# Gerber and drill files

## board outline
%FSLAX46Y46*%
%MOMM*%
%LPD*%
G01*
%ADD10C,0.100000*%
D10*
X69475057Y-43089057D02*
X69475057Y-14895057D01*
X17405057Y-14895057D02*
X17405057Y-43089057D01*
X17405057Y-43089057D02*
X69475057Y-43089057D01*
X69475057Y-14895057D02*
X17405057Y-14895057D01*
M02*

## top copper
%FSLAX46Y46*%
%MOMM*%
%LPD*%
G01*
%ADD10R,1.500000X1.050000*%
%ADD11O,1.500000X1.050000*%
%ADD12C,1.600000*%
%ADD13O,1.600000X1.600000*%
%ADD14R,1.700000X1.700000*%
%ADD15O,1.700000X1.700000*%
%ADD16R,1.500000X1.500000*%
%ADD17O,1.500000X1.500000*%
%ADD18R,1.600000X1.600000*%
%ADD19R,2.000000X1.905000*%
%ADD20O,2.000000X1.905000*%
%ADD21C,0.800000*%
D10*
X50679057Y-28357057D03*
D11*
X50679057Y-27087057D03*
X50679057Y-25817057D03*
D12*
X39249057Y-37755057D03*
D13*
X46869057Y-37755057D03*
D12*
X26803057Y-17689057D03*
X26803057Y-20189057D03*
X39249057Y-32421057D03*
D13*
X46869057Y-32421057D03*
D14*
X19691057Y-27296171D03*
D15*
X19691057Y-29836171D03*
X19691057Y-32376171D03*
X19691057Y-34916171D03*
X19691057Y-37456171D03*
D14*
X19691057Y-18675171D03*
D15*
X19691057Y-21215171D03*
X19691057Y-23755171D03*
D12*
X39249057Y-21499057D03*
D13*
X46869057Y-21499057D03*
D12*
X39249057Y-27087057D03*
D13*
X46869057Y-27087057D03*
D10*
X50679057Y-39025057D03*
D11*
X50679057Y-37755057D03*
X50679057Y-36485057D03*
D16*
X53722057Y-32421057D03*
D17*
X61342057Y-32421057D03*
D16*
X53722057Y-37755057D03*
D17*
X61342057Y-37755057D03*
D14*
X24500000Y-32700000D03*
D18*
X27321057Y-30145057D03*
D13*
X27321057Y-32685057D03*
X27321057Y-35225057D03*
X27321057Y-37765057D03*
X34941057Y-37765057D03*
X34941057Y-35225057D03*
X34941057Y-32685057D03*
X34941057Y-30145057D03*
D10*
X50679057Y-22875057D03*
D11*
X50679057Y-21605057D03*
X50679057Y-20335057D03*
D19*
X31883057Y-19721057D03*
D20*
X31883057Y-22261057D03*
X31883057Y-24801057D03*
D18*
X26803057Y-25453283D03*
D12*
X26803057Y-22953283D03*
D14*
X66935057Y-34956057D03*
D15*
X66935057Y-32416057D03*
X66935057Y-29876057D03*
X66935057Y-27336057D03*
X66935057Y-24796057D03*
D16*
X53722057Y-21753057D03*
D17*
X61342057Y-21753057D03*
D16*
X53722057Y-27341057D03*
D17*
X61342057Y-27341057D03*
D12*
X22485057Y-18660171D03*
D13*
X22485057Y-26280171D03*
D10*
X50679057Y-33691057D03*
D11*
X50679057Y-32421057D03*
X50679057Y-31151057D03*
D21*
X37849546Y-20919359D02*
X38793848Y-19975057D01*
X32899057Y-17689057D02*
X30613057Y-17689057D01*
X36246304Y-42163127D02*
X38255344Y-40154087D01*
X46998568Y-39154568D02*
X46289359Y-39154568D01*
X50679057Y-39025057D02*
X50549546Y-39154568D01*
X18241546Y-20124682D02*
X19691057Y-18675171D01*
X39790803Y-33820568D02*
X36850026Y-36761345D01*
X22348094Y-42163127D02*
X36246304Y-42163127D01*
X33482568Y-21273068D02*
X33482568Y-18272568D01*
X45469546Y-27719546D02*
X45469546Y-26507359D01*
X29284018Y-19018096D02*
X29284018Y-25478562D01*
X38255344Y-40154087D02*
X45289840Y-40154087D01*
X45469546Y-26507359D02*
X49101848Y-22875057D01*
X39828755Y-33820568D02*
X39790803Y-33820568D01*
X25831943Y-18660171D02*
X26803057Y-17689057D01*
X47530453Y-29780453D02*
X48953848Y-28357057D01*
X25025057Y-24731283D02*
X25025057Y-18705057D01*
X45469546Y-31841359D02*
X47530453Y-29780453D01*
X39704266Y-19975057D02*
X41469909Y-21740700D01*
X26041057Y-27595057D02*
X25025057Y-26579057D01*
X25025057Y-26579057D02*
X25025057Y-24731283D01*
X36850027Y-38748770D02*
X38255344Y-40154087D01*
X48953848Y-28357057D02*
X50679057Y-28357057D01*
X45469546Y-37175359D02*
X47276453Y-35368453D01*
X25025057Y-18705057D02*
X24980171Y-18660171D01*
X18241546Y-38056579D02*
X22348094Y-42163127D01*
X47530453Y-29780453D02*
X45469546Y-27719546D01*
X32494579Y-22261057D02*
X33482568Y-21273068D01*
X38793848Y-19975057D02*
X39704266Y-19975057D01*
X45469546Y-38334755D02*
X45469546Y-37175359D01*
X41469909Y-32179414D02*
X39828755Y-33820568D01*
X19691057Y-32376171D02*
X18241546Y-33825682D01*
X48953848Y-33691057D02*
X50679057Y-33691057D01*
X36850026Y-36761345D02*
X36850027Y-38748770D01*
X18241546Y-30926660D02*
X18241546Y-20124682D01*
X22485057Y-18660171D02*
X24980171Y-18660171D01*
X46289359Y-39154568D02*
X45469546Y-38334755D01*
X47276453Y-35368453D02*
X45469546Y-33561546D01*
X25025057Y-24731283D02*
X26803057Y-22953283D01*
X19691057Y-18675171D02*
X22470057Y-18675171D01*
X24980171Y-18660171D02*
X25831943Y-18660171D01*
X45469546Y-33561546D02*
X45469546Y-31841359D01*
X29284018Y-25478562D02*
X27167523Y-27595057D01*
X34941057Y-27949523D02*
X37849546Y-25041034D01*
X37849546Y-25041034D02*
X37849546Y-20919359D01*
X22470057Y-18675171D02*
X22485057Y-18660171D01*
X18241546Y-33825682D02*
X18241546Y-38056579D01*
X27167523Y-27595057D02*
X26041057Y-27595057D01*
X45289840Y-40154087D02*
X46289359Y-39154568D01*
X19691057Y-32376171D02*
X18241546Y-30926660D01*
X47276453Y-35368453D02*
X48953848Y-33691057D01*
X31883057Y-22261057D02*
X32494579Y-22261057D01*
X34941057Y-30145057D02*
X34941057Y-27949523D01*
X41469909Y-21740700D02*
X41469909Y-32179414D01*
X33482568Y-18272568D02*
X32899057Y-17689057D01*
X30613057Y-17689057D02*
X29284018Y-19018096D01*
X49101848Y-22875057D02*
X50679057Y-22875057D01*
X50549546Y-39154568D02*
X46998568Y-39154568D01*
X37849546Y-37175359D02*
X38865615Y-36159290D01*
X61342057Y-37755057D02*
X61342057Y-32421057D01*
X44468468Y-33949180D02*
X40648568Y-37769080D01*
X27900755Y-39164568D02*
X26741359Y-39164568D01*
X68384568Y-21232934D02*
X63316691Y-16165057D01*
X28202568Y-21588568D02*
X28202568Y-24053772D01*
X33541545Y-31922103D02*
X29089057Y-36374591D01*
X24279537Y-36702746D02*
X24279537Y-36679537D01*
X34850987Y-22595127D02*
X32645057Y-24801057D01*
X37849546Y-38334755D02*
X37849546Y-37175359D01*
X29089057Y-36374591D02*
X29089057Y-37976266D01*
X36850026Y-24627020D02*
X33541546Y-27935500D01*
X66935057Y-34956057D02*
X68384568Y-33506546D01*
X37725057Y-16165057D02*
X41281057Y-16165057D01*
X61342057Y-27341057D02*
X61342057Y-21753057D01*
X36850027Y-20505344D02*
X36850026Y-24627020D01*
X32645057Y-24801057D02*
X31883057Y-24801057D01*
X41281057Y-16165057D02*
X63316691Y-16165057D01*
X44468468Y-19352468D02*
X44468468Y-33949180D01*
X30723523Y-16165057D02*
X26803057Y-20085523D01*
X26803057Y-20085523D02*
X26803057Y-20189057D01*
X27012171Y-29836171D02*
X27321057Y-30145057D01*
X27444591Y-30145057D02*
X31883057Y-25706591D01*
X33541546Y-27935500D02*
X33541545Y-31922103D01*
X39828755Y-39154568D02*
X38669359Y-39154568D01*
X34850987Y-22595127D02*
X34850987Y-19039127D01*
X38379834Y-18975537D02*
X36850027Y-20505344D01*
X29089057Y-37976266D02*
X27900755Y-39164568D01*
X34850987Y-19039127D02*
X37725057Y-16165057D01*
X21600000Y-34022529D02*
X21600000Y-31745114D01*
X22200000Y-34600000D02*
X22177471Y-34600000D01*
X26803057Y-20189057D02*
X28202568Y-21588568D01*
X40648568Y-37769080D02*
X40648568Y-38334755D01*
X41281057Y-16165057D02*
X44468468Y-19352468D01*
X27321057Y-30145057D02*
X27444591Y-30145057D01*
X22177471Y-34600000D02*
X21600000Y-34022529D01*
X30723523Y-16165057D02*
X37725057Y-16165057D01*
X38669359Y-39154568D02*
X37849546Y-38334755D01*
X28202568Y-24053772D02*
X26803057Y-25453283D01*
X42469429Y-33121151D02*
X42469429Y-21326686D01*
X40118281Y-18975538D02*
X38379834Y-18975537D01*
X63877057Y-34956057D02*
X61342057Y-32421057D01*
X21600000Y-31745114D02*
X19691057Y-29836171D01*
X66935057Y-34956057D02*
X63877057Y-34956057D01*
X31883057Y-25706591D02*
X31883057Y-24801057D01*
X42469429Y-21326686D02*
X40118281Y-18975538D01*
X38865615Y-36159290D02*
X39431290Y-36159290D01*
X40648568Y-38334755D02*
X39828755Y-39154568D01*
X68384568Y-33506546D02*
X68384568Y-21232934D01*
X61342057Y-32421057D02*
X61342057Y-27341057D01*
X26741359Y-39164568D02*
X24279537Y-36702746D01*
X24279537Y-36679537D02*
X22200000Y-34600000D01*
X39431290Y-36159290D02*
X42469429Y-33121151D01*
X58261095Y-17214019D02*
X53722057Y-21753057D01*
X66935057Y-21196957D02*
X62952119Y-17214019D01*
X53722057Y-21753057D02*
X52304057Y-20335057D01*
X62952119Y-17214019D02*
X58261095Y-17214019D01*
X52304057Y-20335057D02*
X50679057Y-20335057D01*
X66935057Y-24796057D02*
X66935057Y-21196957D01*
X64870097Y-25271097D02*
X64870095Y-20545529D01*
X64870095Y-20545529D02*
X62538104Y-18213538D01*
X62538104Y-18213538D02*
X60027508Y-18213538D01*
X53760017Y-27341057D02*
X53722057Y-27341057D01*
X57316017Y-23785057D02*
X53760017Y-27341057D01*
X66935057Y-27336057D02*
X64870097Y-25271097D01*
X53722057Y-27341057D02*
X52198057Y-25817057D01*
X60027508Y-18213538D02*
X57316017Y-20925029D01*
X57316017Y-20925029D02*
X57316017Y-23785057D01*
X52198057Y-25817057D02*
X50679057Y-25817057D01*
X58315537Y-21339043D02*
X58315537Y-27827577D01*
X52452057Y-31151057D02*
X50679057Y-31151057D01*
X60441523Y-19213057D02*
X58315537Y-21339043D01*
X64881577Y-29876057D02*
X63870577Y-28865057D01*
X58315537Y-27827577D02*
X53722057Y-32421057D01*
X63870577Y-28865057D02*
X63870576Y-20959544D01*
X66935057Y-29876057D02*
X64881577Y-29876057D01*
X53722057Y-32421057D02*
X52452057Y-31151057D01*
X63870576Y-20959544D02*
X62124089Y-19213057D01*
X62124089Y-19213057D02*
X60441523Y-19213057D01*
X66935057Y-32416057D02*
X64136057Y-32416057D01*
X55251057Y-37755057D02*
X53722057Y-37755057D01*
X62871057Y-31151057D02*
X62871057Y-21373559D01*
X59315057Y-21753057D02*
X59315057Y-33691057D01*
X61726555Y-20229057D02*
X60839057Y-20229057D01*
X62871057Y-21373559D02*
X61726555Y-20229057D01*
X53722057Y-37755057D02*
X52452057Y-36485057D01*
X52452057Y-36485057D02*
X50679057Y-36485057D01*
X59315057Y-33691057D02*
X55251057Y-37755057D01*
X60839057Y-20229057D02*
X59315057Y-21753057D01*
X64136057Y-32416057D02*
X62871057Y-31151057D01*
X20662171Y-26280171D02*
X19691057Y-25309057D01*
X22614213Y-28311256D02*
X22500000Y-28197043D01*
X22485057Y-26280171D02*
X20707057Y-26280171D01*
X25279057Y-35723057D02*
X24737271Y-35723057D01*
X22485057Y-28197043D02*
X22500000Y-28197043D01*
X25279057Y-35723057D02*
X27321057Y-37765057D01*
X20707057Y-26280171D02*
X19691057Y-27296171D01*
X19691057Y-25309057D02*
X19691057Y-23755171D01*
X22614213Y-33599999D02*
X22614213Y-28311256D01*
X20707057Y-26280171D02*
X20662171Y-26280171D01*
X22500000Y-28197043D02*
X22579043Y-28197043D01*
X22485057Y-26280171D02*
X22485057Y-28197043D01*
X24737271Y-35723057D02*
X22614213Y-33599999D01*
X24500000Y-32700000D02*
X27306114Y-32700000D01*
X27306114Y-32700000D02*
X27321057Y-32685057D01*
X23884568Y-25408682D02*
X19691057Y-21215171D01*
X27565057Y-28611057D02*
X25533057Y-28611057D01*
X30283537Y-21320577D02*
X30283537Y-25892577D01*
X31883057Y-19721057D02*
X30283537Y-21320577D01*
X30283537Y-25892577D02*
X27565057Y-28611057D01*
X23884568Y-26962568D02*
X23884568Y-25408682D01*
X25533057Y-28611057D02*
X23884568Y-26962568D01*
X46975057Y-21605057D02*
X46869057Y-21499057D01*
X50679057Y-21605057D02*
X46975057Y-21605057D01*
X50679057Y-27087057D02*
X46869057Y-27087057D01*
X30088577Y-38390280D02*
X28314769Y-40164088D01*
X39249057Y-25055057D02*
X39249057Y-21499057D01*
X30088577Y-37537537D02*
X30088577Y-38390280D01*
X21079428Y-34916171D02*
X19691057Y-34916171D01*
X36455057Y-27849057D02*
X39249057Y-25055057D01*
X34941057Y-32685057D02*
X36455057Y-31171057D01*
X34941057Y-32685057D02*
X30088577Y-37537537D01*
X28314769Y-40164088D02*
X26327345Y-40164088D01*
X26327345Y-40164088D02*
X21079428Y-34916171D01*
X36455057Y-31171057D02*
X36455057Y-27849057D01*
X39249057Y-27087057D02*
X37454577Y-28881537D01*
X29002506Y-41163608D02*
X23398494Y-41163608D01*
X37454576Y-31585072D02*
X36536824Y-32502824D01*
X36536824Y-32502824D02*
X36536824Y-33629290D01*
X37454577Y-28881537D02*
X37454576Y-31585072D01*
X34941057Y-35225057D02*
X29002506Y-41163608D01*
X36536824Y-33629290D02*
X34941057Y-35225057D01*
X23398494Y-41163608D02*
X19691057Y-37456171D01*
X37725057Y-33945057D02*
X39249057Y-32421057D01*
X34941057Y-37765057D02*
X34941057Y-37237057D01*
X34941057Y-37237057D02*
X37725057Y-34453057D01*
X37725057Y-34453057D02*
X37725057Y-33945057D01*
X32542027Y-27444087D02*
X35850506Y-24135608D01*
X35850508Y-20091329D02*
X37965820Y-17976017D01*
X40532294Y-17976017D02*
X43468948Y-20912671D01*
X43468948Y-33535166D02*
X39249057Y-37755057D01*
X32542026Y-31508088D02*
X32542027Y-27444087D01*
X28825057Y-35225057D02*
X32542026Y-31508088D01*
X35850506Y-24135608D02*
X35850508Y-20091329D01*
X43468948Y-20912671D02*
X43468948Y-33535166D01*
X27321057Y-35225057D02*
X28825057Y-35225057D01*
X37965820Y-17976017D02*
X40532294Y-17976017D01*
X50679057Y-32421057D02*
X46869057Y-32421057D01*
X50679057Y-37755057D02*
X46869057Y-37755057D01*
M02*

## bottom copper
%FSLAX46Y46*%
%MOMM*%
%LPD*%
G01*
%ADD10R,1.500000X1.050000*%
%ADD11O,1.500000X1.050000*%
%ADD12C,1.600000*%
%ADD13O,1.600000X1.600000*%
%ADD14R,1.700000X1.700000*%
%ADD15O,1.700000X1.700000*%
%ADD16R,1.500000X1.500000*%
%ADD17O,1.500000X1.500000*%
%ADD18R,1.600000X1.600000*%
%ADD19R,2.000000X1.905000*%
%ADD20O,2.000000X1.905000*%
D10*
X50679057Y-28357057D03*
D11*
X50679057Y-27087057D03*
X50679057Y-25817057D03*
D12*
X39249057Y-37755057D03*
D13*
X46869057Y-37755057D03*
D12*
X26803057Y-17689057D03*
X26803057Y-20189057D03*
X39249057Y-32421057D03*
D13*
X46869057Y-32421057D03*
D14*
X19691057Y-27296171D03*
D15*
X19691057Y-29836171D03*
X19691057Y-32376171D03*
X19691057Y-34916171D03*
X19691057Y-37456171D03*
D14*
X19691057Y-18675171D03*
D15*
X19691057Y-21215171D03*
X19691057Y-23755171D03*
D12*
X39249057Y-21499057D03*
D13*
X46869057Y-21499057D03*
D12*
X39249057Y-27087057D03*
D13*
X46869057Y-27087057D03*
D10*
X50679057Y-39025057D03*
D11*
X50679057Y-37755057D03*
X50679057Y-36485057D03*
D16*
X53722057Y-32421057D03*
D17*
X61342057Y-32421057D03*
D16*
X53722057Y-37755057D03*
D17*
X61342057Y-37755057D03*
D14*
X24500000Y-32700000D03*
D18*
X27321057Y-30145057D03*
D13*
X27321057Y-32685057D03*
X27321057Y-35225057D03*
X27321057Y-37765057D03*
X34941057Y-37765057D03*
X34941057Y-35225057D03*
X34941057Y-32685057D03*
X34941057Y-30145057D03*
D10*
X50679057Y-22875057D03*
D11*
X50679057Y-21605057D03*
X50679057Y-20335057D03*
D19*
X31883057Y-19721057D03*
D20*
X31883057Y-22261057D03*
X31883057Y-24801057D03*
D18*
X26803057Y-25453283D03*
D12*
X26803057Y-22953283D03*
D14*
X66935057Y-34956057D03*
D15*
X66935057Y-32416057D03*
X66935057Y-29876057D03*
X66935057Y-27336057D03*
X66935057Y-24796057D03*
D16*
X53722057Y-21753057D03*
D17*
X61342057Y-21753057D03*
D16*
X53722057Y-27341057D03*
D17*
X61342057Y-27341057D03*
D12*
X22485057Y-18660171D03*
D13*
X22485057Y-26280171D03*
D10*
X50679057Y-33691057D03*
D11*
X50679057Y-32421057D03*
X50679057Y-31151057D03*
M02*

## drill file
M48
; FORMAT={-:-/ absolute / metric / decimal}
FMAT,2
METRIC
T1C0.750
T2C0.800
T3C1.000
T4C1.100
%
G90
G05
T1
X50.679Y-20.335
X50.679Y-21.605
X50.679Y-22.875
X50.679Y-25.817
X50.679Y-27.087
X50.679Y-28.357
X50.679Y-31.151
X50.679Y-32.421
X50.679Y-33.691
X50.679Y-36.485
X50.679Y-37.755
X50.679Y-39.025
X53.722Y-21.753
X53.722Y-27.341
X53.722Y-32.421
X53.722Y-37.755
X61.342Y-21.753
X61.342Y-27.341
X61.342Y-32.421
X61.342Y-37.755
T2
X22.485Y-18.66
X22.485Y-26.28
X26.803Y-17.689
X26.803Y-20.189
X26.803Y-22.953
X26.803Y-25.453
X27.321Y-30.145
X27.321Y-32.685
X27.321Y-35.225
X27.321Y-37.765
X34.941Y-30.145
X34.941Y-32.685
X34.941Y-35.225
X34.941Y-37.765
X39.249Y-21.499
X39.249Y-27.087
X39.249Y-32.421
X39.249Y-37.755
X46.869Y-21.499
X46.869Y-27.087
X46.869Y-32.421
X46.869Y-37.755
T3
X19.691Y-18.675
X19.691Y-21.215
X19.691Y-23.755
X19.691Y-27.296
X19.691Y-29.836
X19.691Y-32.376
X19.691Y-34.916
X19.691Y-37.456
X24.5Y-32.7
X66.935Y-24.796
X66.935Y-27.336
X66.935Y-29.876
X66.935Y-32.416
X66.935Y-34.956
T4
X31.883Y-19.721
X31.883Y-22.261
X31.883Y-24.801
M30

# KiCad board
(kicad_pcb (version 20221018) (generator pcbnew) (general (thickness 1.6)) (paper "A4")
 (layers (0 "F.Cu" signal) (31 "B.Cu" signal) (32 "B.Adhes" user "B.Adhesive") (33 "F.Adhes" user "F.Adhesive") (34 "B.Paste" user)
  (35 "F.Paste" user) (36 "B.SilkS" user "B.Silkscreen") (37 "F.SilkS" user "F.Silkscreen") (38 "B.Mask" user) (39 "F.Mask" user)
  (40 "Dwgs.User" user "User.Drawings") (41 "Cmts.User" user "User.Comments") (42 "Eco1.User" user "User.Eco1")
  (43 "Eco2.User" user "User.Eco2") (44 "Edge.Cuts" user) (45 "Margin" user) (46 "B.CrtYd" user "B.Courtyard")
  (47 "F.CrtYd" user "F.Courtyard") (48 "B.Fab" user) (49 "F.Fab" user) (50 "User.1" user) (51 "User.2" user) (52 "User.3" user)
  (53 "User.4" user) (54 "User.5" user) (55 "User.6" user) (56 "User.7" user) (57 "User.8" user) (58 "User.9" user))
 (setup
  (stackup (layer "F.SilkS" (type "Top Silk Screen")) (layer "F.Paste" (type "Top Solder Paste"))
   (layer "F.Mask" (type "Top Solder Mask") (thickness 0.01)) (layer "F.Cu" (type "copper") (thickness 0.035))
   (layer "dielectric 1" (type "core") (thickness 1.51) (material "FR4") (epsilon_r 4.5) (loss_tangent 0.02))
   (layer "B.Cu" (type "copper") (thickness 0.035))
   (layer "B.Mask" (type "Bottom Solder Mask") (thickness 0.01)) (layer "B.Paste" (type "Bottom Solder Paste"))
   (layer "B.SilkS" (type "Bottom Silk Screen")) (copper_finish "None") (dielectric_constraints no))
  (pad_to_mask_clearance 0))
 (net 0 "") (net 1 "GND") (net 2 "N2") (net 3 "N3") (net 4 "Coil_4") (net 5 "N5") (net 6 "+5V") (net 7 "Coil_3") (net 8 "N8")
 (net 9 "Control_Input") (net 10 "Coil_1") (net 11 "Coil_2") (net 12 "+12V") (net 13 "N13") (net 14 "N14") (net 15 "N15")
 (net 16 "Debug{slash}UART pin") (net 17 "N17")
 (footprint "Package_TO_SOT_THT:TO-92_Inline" (layer "F.Cu") (at 50.679057 28.357057 90)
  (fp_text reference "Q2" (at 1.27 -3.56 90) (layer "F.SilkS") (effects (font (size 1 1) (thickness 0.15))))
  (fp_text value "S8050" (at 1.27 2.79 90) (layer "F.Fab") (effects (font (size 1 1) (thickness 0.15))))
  (pad "1" thru_hole rect (at 0 0 90) (size 1.05 1.5) (drill 0.75) (layers "*.Cu" "*.Mask") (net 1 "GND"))
  (pad "2" thru_hole oval (at 1.27 0 90) (size 1.05 1.5) (drill 0.75) (layers "*.Cu" "*.Mask") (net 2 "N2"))
  (pad "3" thru_hole oval (at 2.54 0 90) (size 1.05 1.5) (drill 0.75) (layers "*.Cu" "*.Mask") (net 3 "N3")))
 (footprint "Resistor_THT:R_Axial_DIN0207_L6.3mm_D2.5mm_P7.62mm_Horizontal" (layer "F.Cu") (at 39.249057 37.755057)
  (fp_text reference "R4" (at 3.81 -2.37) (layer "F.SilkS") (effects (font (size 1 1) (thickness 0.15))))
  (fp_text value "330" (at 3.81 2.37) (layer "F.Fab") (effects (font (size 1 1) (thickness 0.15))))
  (pad "1" thru_hole circle (at 0 0) (size 1.6 1.6) (drill 0.8) (layers "*.Cu" "*.Mask") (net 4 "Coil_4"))
  (pad "2" thru_hole oval (at 7.62 0) (size 1.6 1.6) (drill 0.8) (layers "*.Cu" "*.Mask") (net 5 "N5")))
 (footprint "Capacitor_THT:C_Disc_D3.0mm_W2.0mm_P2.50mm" (layer "F.Cu") (at 26.803057 17.689057 -90)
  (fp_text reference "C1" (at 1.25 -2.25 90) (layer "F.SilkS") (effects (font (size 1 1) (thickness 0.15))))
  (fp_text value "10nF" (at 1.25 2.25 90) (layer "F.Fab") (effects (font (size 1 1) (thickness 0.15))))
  (pad "1" thru_hole circle (at 0 0 270) (size 1.6 1.6) (drill 0.8) (layers "*.Cu" "*.Mask") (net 1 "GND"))
  (pad "2" thru_hole circle (at 2.5 0 270) (size 1.6 1.6) (drill 0.8) (layers "*.Cu" "*.Mask") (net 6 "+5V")))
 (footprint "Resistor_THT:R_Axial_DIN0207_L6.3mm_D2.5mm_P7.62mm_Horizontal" (layer "F.Cu") (at 39.249057 32.421057)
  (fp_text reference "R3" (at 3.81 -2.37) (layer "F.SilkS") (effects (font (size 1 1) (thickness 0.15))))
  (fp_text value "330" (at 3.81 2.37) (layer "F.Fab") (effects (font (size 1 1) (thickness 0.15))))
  (pad "1" thru_hole circle (at 0 0) (size 1.6 1.6) (drill 0.8) (layers "*.Cu" "*.Mask") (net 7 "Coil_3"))
  (pad "2" thru_hole oval (at 7.62 0) (size 1.6 1.6) (drill 0.8) (layers "*.Cu" "*.Mask") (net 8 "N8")))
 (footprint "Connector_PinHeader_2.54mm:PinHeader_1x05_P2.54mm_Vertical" (layer "F.Cu") (at 19.691057 27.296171)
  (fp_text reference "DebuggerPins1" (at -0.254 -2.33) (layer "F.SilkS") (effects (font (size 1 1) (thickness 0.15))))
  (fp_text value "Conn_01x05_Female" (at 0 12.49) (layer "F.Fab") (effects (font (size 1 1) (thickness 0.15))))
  (pad "1" thru_hole rect (at 0 0) (size 1.7 1.7) (drill 1) (layers "*.Cu" "*.Mask") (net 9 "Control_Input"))
  (pad "2" thru_hole oval (at 0 2.54) (size 1.7 1.7) (drill 1) (layers "*.Cu" "*.Mask") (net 6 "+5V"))
  (pad "3" thru_hole oval (at 0 5.08) (size 1.7 1.7) (drill 1) (layers "*.Cu" "*.Mask") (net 1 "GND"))
  (pad "4" thru_hole oval (at 0 7.62) (size 1.7 1.7) (drill 1) (layers "*.Cu" "*.Mask") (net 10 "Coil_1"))
  (pad "5" thru_hole oval (at 0 10.16) (size 1.7 1.7) (drill 1) (layers "*.Cu" "*.Mask") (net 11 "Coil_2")))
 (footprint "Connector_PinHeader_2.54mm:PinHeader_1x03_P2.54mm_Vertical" (layer "F.Cu") (at 19.691057 18.675171)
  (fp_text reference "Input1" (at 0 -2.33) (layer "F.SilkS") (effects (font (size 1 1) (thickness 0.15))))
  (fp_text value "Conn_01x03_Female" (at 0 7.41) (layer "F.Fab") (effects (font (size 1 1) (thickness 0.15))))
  (pad "1" thru_hole rect (at 0 0) (size 1.7 1.7) (drill 1) (layers "*.Cu" "*.Mask") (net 1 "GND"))
  (pad "2" thru_hole oval (at 0 2.54) (size 1.7 1.7) (drill 1) (layers "*.Cu" "*.Mask") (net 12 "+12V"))
  (pad "3" thru_hole oval (at 0 5.08) (size 1.7 1.7) (drill 1) (layers "*.Cu" "*.Mask") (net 9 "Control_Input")))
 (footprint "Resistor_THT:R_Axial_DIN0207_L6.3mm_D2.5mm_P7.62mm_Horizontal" (layer "F.Cu") (at 39.249057 21.499057)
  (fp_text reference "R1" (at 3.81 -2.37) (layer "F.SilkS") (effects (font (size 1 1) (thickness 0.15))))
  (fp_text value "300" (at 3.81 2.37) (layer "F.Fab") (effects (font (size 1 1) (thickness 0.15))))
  (pad "1" thru_hole circle (at 0 0) (size 1.6 1.6) (drill 0.8) (layers "*.Cu" "*.Mask") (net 10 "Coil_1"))
  (pad "2" thru_hole oval (at 7.62 0) (size 1.6 1.6) (drill 0.8) (layers "*.Cu" "*.Mask") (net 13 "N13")))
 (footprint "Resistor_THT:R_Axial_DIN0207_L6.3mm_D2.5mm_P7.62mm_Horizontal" (layer "F.Cu") (at 39.249057 27.087057)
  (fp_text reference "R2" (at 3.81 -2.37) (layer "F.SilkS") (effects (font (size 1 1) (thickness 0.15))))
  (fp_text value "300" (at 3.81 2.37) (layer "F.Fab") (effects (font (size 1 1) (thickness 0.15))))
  (pad "1" thru_hole circle (at 0 0) (size 1.6 1.6) (drill 0.8) (layers "*.Cu" "*.Mask") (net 11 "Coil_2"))
  (pad "2" thru_hole oval (at 7.62 0) (size 1.6 1.6) (drill 0.8) (layers "*.Cu" "*.Mask") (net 2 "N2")))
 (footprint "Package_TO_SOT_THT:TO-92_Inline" (layer "F.Cu") (at 50.679057 39.025057 90)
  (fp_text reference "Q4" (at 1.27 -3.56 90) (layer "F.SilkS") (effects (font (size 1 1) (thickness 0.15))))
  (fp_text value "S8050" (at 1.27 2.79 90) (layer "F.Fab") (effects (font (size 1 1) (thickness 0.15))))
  (pad "1" thru_hole rect (at 0 0 90) (size 1.05 1.5) (drill 0.75) (layers "*.Cu" "*.Mask") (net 1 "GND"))
  (pad "2" thru_hole oval (at 1.27 0 90) (size 1.05 1.5) (drill 0.75) (layers "*.Cu" "*.Mask") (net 5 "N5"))
  (pad "3" thru_hole oval (at 2.54 0 90) (size 1.05 1.5) (drill 0.75) (layers "*.Cu" "*.Mask") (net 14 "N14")))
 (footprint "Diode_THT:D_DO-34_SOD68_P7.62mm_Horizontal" (layer "F.Cu") (at 53.722057 32.421057)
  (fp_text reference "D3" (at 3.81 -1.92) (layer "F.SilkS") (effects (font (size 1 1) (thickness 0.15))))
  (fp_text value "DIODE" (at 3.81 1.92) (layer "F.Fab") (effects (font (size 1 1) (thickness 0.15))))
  (pad "1" thru_hole rect (at 0 0) (size 1.5 1.5) (drill 0.75) (layers "*.Cu" "*.Mask") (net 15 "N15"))
  (pad "2" thru_hole oval (at 7.62 0) (size 1.5 1.5) (drill 0.75) (layers "*.Cu" "*.Mask") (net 6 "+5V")))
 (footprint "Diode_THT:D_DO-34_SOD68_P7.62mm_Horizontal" (layer "F.Cu") (at 53.722057 37.755057)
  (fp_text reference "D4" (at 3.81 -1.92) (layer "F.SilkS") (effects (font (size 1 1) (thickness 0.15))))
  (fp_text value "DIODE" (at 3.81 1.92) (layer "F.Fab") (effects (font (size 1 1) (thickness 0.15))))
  (pad "1" thru_hole rect (at 0 0) (size 1.5 1.5) (drill 0.75) (layers "*.Cu" "*.Mask") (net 14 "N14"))
  (pad "2" thru_hole oval (at 7.62 0) (size 1.5 1.5) (drill 0.75) (layers "*.Cu" "*.Mask") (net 6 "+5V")))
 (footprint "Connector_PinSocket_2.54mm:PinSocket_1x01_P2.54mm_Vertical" (layer "F.Cu") (at 24.5 32.7)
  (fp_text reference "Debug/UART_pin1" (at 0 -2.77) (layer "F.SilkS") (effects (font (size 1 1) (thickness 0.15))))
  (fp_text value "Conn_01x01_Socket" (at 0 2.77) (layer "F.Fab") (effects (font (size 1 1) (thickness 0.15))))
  (pad "1" thru_hole rect (at 0 0) (size 1.7 1.7) (drill 1) (layers "*.Cu" "*.Mask") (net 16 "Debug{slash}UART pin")))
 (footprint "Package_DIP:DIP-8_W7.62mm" (layer "F.Cu") (at 27.321057 30.145057)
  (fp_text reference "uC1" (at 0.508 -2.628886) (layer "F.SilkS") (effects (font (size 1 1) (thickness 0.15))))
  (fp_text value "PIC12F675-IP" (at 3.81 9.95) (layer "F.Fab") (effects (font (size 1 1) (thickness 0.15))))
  (pad "1" thru_hole rect (at 0 0) (size 1.6 1.6) (drill 0.8) (layers "*.Cu" "*.Mask") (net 6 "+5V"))
  (pad "2" thru_hole oval (at 0 2.54) (size 1.6 1.6) (drill 0.8) (layers "*.Cu" "*.Mask") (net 16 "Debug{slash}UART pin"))
  (pad "3" thru_hole oval (at 0 5.08) (size 1.6 1.6) (drill 0.8) (layers "*.Cu" "*.Mask") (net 4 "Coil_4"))
  (pad "4" thru_hole oval (at 0 7.62) (size 1.6 1.6) (drill 0.8) (layers "*.Cu" "*.Mask") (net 9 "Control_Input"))
  (pad "5" thru_hole oval (at 7.62 7.62) (size 1.6 1.6) (drill 0.8) (layers "*.Cu" "*.Mask") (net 7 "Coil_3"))
  (pad "6" thru_hole oval (at 7.62 5.08) (size 1.6 1.6) (drill 0.8) (layers "*.Cu" "*.Mask") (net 11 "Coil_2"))
  (pad "7" thru_hole oval (at 7.62 2.54) (size 1.6 1.6) (drill 0.8) (layers "*.Cu" "*.Mask") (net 10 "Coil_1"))
  (pad "8" thru_hole oval (at 7.62 0) (size 1.6 1.6) (drill 0.8) (layers "*.Cu" "*.Mask") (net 1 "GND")))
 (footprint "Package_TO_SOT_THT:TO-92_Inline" (layer "F.Cu") (at 50.679057 22.875057 90)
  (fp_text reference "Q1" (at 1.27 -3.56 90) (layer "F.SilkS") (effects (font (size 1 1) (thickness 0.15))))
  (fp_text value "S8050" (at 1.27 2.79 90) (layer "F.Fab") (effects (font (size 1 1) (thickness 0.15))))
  (pad "1" thru_hole rect (at 0 0 90) (size 1.05 1.5) (drill 0.75) (layers "*.Cu" "*.Mask") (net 1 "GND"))
  (pad "2" thru_hole oval (at 1.27 0 90) (size 1.05 1.5) (drill 0.75) (layers "*.Cu" "*.Mask") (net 13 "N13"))
  (pad "3" thru_hole oval (at 2.54 0 90) (size 1.05 1.5) (drill 0.75) (layers "*.Cu" "*.Mask") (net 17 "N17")))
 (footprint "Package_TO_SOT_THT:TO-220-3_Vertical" (layer "F.Cu") (at 31.883057 19.721057 -90)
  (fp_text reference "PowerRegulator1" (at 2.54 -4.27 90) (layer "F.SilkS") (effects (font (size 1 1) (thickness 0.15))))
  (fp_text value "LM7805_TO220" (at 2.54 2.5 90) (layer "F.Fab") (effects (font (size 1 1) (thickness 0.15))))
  (pad "1" thru_hole rect (at 0 0 270) (size 1.905 2) (drill 1.1) (layers "*.Cu" "*.Mask") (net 12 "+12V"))
  (pad "2" thru_hole oval (at 2.54 0 270) (size 1.905 2) (drill 1.1) (layers "*.Cu" "*.Mask") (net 1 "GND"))
  (pad "3" thru_hole oval (at 5.08 0 270) (size 1.905 2) (drill 1.1) (layers "*.Cu" "*.Mask") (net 6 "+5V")))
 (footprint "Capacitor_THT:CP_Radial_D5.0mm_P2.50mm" (layer "F.Cu") (at 26.803057 25.453283 90)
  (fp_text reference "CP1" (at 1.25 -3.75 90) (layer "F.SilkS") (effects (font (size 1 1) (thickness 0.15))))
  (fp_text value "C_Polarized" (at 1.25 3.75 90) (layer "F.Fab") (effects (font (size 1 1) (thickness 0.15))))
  (pad "1" thru_hole rect (at 0 0 90) (size 1.6 1.6) (drill 0.8) (layers "*.Cu" "*.Mask") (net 6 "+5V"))
  (pad "2" thru_hole circle (at 2.5 0 90) (size 1.6 1.6) (drill 0.8) (layers "*.Cu" "*.Mask") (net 1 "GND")))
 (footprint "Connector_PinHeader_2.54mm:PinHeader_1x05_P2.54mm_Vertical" (layer "F.Cu") (at 66.935057 34.956057 180)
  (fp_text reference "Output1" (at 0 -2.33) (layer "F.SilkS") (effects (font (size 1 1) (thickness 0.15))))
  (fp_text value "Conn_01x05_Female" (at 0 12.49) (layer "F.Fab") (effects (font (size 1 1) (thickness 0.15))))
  (pad "1" thru_hole rect (at 0 0 180) (size 1.7 1.7) (drill 1) (layers "*.Cu" "*.Mask") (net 6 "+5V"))
  (pad "2" thru_hole oval (at 0 2.54 180) (size 1.7 1.7) (drill 1) (layers "*.Cu" "*.Mask") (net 14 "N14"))
  (pad "3" thru_hole oval (at 0 5.08 180) (size 1.7 1.7) (drill 1) (layers "*.Cu" "*.Mask") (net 15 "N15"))
  (pad "4" thru_hole oval (at 0 7.62 180) (size 1.7 1.7) (drill 1) (layers "*.Cu" "*.Mask") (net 3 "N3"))
  (pad "5" thru_hole oval (at 0 10.16 180) (size 1.7 1.7) (drill 1) (layers "*.Cu" "*.Mask") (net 17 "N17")))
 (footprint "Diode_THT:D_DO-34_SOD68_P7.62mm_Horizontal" (layer "F.Cu") (at 53.722057 21.753057)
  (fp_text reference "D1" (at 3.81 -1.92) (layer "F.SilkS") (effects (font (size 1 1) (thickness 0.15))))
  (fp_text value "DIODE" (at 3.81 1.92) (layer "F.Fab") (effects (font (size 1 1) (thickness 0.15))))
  (pad "1" thru_hole rect (at 0 0) (size 1.5 1.5) (drill 0.75) (layers "*.Cu" "*.Mask") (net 17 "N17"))
  (pad "2" thru_hole oval (at 7.62 0) (size 1.5 1.5) (drill 0.75) (layers "*.Cu" "*.Mask") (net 6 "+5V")))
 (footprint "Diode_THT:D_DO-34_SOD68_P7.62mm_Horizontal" (layer "F.Cu") (at 53.722057 27.341057)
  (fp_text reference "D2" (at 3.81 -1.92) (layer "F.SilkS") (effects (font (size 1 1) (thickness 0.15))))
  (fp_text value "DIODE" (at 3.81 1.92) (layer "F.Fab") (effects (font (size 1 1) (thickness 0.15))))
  (pad "1" thru_hole rect (at 0 0) (size 1.5 1.5) (drill 0.75) (layers "*.Cu" "*.Mask") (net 3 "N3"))
  (pad "2" thru_hole oval (at 7.62 0) (size 1.5 1.5) (drill 0.75) (layers "*.Cu" "*.Mask") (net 6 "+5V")))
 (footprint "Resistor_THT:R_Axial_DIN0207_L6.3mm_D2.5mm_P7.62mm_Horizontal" (layer "F.Cu") (at 22.485057 18.660171 -90)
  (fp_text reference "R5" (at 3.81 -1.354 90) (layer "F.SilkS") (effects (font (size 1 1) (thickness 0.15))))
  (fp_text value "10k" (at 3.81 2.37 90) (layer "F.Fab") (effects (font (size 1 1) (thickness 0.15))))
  (pad "1" thru_hole circle (at 0 0 270) (size 1.6 1.6) (drill 0.8) (layers "*.Cu" "*.Mask") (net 1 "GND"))
  (pad "2" thru_hole oval (at 7.62 0 270) (size 1.6 1.6) (drill 0.8) (layers "*.Cu" "*.Mask") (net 9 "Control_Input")))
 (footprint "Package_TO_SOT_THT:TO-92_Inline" (layer "F.Cu") (at 50.679057 33.691057 90)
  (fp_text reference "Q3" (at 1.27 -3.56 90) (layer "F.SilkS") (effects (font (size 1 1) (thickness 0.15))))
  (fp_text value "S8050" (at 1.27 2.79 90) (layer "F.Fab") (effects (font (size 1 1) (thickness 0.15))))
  (pad "1" thru_hole rect (at 0 0 90) (size 1.05 1.5) (drill 0.75) (layers "*.Cu" "*.Mask") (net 1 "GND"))
  (pad "2" thru_hole oval (at 1.27 0 90) (size 1.05 1.5) (drill 0.75) (layers "*.Cu" "*.Mask") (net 8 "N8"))
  (pad "3" thru_hole oval (at 2.54 0 90) (size 1.05 1.5) (drill 0.75) (layers "*.Cu" "*.Mask") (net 15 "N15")))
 (gr_line (start 69.475057 43.089057) (end 69.475057 14.895057) (stroke (width 0.1) (type solid)) (layer "Edge.Cuts"))
 (gr_line (start 17.405057 14.895057) (end 17.405057 43.089057) (stroke (width 0.1) (type solid)) (layer "Edge.Cuts"))
 (gr_line (start 17.405057 43.089057) (end 69.475057 43.089057) (stroke (width 0.1) (type solid)) (layer "Edge.Cuts"))
 (gr_line (start 69.475057 14.895057) (end 17.405057 14.895057) (stroke (width 0.1) (type solid)) (layer "Edge.Cuts"))
 (segment (start 37.849546 20.919359) (end 38.793848 19.975057) (width 0.8) (layer "F.Cu") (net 1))
 (segment (start 32.899057 17.689057) (end 30.613057 17.689057) (width 0.8) (layer "F.Cu") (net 1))
 (segment (start 36.246304 42.163127) (end 38.255344 40.154087) (width 0.8) (layer "F.Cu") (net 1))
 (segment (start 46.998568 39.154568) (end 46.289359 39.154568) (width 0.8) (layer "F.Cu") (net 1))
 (segment (start 50.679057 39.025057) (end 50.549546 39.154568) (width 0.8) (layer "F.Cu") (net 1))
 (segment (start 18.241546 20.124682) (end 19.691057 18.675171) (width 0.8) (layer "F.Cu") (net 1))
 (segment (start 39.790803 33.820568) (end 36.850026 36.761345) (width 0.8) (layer "F.Cu") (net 1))
 (segment (start 22.348094 42.163127) (end 36.246304 42.163127) (width 0.8) (layer "F.Cu") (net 1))
 (segment (start 33.482568 21.273068) (end 33.482568 18.272568) (width 0.8) (layer "F.Cu") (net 1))
 (segment (start 45.469546 27.719546) (end 45.469546 26.507359) (width 0.8) (layer "F.Cu") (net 1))
 (segment (start 29.284018 19.018096) (end 29.284018 25.478562) (width 0.8) (layer "F.Cu") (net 1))
 (segment (start 38.255344 40.154087) (end 45.28984 40.154087) (width 0.8) (layer "F.Cu") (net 1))
 (segment (start 45.469546 26.507359) (end 49.101848 22.875057) (width 0.8) (layer "F.Cu") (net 1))
 (segment (start 39.828755 33.820568) (end 39.790803 33.820568) (width 0.8) (layer "F.Cu") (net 1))
 (segment (start 25.831943 18.660171) (end 26.803057 17.689057) (width 0.8) (layer "F.Cu") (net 1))
 (segment (start 47.530453 29.780453) (end 48.953848 28.357057) (width 0.8) (layer "F.Cu") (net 1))
 (segment (start 25.025057 24.731283) (end 25.025057 18.705057) (width 0.8) (layer "F.Cu") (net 1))
 (segment (start 45.469546 31.841359) (end 47.530453 29.780453) (width 0.8) (layer "F.Cu") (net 1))
 (segment (start 39.704266 19.975057) (end 41.469909 21.7407) (width 0.8) (layer "F.Cu") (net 1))
 (segment (start 26.041057 27.595057) (end 25.025057 26.579057) (width 0.8) (layer "F.Cu") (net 1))
 (segment (start 25.025057 26.579057) (end 25.025057 24.731283) (width 0.8) (layer "F.Cu") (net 1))
 (segment (start 36.850027 38.74877) (end 38.255344 40.154087) (width 0.8) (layer "F.Cu") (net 1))
 (segment (start 48.953848 28.357057) (end 50.679057 28.357057) (width 0.8) (layer "F.Cu") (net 1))
 (segment (start 45.469546 37.175359) (end 47.276453 35.368453) (width 0.8) (layer "F.Cu") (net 1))
 (segment (start 25.025057 18.705057) (end 24.980171 18.660171) (width 0.8) (layer "F.Cu") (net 1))
 (segment (start 18.241546 38.056579) (end 22.348094 42.163127) (width 0.8) (layer "F.Cu") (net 1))
 (segment (start 47.530453 29.780453) (end 45.469546 27.719546) (width 0.8) (layer "F.Cu") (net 1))
 (segment (start 32.494579 22.261057) (end 33.482568 21.273068) (width 0.8) (layer "F.Cu") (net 1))
 (segment (start 38.793848 19.975057) (end 39.704266 19.975057) (width 0.8) (layer "F.Cu") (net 1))
 (segment (start 45.469546 38.334755) (end 45.469546 37.175359) (width 0.8) (layer "F.Cu") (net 1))
 (segment (start 41.469909 32.179414) (end 39.828755 33.820568) (width 0.8) (layer "F.Cu") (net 1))
 (segment (start 19.691057 32.376171) (end 18.241546 33.825682) (width 0.8) (layer "F.Cu") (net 1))
 (segment (start 48.953848 33.691057) (end 50.679057 33.691057) (width 0.8) (layer "F.Cu") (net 1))
 (segment (start 36.850026 36.761345) (end 36.850027 38.74877) (width 0.8) (layer "F.Cu") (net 1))
 (segment (start 18.241546 30.92666) (end 18.241546 20.124682) (width 0.8) (layer "F.Cu") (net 1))
 (segment (start 22.485057 18.660171) (end 24.980171 18.660171) (width 0.8) (layer "F.Cu") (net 1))
 (segment (start 46.289359 39.154568) (end 45.469546 38.334755) (width 0.8) (layer "F.Cu") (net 1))
 (segment (start 47.276453 35.368453) (end 45.469546 33.561546) (width 0.8) (layer "F.Cu") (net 1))
 (segment (start 25.025057 24.731283) (end 26.803057 22.953283) (width 0.8) (layer "F.Cu") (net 1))
 (segment (start 19.691057 18.675171) (end 22.470057 18.675171) (width 0.8) (layer "F.Cu") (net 1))
 (segment (start 24.980171 18.660171) (end 25.831943 18.660171) (width 0.8) (layer "F.Cu") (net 1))
 (segment (start 45.469546 33.561546) (end 45.469546 31.841359) (width 0.8) (layer "F.Cu") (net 1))
 (segment (start 29.284018 25.478562) (end 27.167523 27.595057) (width 0.8) (layer "F.Cu") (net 1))
 (segment (start 34.941057 27.949523) (end 37.849546 25.041034) (width 0.8) (layer "F.Cu") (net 1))
 (segment (start 37.849546 25.041034) (end 37.849546 20.919359) (width 0.8) (layer "F.Cu") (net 1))
 (segment (start 22.470057 18.675171) (end 22.485057 18.660171) (width 0.8) (layer "F.Cu") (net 1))
 (segment (start 18.241546 33.825682) (end 18.241546 38.056579) (width 0.8) (layer "F.Cu") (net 1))
 (segment (start 27.167523 27.595057) (end 26.041057 27.595057) (width 0.8) (layer "F.Cu") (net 1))
 (segment (start 45.28984 40.154087) (end 46.289359 39.154568) (width 0.8) (layer "F.Cu") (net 1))
 (segment (start 19.691057 32.376171) (end 18.241546 30.92666) (width 0.8) (layer "F.Cu") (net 1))
 (segment (start 47.276453 35.368453) (end 48.953848 33.691057) (width 0.8) (layer "F.Cu") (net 1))
 (segment (start 31.883057 22.261057) (end 32.494579 22.261057) (width 0.8) (layer "F.Cu") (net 1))
 (segment (start 34.941057 30.145057) (end 34.941057 27.949523) (width 0.8) (layer "F.Cu") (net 1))
 (segment (start 41.469909 21.7407) (end 41.469909 32.179414) (width 0.8) (layer "F.Cu") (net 1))
 (segment (start 33.482568 18.272568) (end 32.899057 17.689057) (width 0.8) (layer "F.Cu") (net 1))
 (segment (start 30.613057 17.689057) (end 29.284018 19.018096) (width 0.8) (layer "F.Cu") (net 1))
 (segment (start 49.101848 22.875057) (end 50.679057 22.875057) (width 0.8) (layer "F.Cu") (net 1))
 (segment (start 50.549546 39.154568) (end 46.998568 39.154568) (width 0.8) (layer "F.Cu") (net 1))
 (segment (start 37.849546 37.175359) (end 38.865615 36.15929) (width 0.8) (layer "F.Cu") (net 6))
 (segment (start 61.342057 37.755057) (end 61.342057 32.421057) (width 0.8) (layer "F.Cu") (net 6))
 (segment (start 44.468468 33.94918) (end 40.648568 37.76908) (width 0.8) (layer "F.Cu") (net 6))
 (segment (start 27.900755 39.164568) (end 26.741359 39.164568) (width 0.8) (layer "F.Cu") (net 6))
 (segment (start 68.384568 21.232934) (end 63.316691 16.165057) (width 0.8) (layer "F.Cu") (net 6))
 (segment (start 28.202568 21.588568) (end 28.202568 24.053772) (width 0.8) (layer "F.Cu") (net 6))
 (segment (start 33.541545 31.922103) (end 29.089057 36.374591) (width 0.8) (layer "F.Cu") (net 6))
 (segment (start 24.279537 36.702746) (end 24.279537 36.679537) (width 0.8) (layer "F.Cu") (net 6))
 (segment (start 34.850987 22.595127) (end 32.645057 24.801057) (width 0.8) (layer "F.Cu") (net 6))
 (segment (start 37.849546 38.334755) (end 37.849546 37.175359) (width 0.8) (layer "F.Cu") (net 6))
 (segment (start 29.089057 36.374591) (end 29.089057 37.976266) (width 0.8) (layer "F.Cu") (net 6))
 (segment (start 36.850026 24.62702) (end 33.541546 27.9355) (width 0.8) (layer "F.Cu") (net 6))
 (segment (start 66.935057 34.956057) (end 68.384568 33.506546) (width 0.8) (layer "F.Cu") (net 6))
 (segment (start 37.725057 16.165057) (end 41.281057 16.165057) (width 0.8) (layer "F.Cu") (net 6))
 (segment (start 61.342057 27.341057) (end 61.342057 21.753057) (width 0.8) (layer "F.Cu") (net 6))
 (segment (start 36.850027 20.505344) (end 36.850026 24.62702) (width 0.8) (layer "F.Cu") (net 6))
 (segment (start 32.645057 24.801057) (end 31.883057 24.801057) (width 0.8) (layer "F.Cu") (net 6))
 (segment (start 41.281057 16.165057) (end 63.316691 16.165057) (width 0.8) (layer "F.Cu") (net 6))
 (segment (start 44.468468 19.352468) (end 44.468468 33.94918) (width 0.8) (layer "F.Cu") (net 6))
 (segment (start 30.723523 16.165057) (end 26.803057 20.085523) (width 0.8) (layer "F.Cu") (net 6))
 (segment (start 26.803057 20.085523) (end 26.803057 20.189057) (width 0.8) (layer "F.Cu") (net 6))
 (segment (start 27.012171 29.836171) (end 27.321057 30.145057) (width 0.8) (layer "F.Cu") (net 6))
 (segment (start 27.444591 30.145057) (end 31.883057 25.706591) (width 0.8) (layer "F.Cu") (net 6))
 (segment (start 33.541546 27.9355) (end 33.541545 31.922103) (width 0.8) (layer "F.Cu") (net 6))
 (segment (start 39.828755 39.154568) (end 38.669359 39.154568) (width 0.8) (layer "F.Cu") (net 6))
 (segment (start 34.850987 22.595127) (end 34.850987 19.039127) (width 0.8) (layer "F.Cu") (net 6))
 (segment (start 38.379834 18.975537) (end 36.850027 20.505344) (width 0.8) (layer "F.Cu") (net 6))
 (segment (start 29.089057 37.976266) (end 27.900755 39.164568) (width 0.8) (layer "F.Cu") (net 6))
 (segment (start 34.850987 19.039127) (end 37.725057 16.165057) (width 0.8) (layer "F.Cu") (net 6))
 (segment (start 21.6 34.022529) (end 21.6 31.745114) (width 0.8) (layer "F.Cu") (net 6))
 (segment (start 22.2 34.6) (end 22.177471 34.6) (width 0.8) (layer "F.Cu") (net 6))
 (segment (start 26.803057 20.189057) (end 28.202568 21.588568) (width 0.8) (layer "F.Cu") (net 6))
 (segment (start 40.648568 37.76908) (end 40.648568 38.334755) (width 0.8) (layer "F.Cu") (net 6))
 (segment (start 41.281057 16.165057) (end 44.468468 19.352468) (width 0.8) (layer "F.Cu") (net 6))
 (segment (start 27.321057 30.145057) (end 27.444591 30.145057) (width 0.8) (layer "F.Cu") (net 6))
 (segment (start 22.177471 34.6) (end 21.6 34.022529) (width 0.8) (layer "F.Cu") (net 6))
 (segment (start 30.723523 16.165057) (end 37.725057 16.165057) (width 0.8) (layer "F.Cu") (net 6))
 (segment (start 38.669359 39.154568) (end 37.849546 38.334755) (width 0.8) (layer "F.Cu") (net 6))
 (segment (start 28.202568 24.053772) (end 26.803057 25.453283) (width 0.8) (layer "F.Cu") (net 6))
 (segment (start 42.469429 33.121151) (end 42.469429 21.326686) (width 0.8) (layer "F.Cu") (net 6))
 (segment (start 40.118281 18.975538) (end 38.379834 18.975537) (width 0.8) (layer "F.Cu") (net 6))
 (segment (start 63.877057 34.956057) (end 61.342057 32.421057) (width 0.8) (layer "F.Cu") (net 6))
 (segment (start 21.6 31.745114) (end 19.691057 29.836171) (width 0.8) (layer "F.Cu") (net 6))
 (segment (start 66.935057 34.956057) (end 63.877057 34.956057) (width 0.8) (layer "F.Cu") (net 6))
 (segment (start 31.883057 25.706591) (end 31.883057 24.801057) (width 0.8) (layer "F.Cu") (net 6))
 (segment (start 42.469429 21.326686) (end 40.118281 18.975538) (width 0.8) (layer "F.Cu") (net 6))
 (segment (start 38.865615 36.15929) (end 39.43129 36.15929) (width 0.8) (layer "F.Cu") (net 6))
 (segment (start 40.648568 38.334755) (end 39.828755 39.154568) (width 0.8) (layer "F.Cu") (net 6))
 (segment (start 68.384568 33.506546) (end 68.384568 21.232934) (width 0.8) (layer "F.Cu") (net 6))
 (segment (start 61.342057 32.421057) (end 61.342057 27.341057) (width 0.8) (layer "F.Cu") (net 6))
 (segment (start 26.741359 39.164568) (end 24.279537 36.702746) (width 0.8) (layer "F.Cu") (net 6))
 (segment (start 24.279537 36.679537) (end 22.2 34.6) (width 0.8) (layer "F.Cu") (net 6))
 (segment (start 39.43129 36.15929) (end 42.469429 33.121151) (width 0.8) (layer "F.Cu") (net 6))
 (segment (start 58.261095 17.214019) (end 53.722057 21.753057) (width 0.8) (layer "F.Cu") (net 17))
 (segment (start 66.935057 21.196957) (end 62.952119 17.214019) (width 0.8) (layer "F.Cu") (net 17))
 (segment (start 53.722057 21.753057) (end 52.304057 20.335057) (width 0.8) (layer "F.Cu") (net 17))
 (segment (start 62.952119 17.214019) (end 58.261095 17.214019) (width 0.8) (layer "F.Cu") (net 17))
 (segment (start 52.304057 20.335057) (end 50.679057 20.335057) (width 0.8) (layer "F.Cu") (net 17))
 (segment (start 66.935057 24.796057) (end 66.935057 21.196957) (width 0.8) (layer "F.Cu") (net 17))
 (segment (start 64.870097 25.271097) (end 64.870095 20.545529) (width 0.8) (layer "F.Cu") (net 3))
 (segment (start 64.870095 20.545529) (end 62.538104 18.213538) (width 0.8) (layer "F.Cu") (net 3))
 (segment (start 62.538104 18.213538) (end 60.027508 18.213538) (width 0.8) (layer "F.Cu") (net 3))
 (segment (start 53.760017 27.341057) (end 53.722057 27.341057) (width 0.8) (layer "F.Cu") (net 3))
 (segment (start 57.316017 23.785057) (end 53.760017 27.341057) (width 0.8) (layer "F.Cu") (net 3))
 (segment (start 66.935057 27.336057) (end 64.870097 25.271097) (width 0.8) (layer "F.Cu") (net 3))
 (segment (start 53.722057 27.341057) (end 52.198057 25.817057) (width 0.8) (layer "F.Cu") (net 3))
 (segment (start 60.027508 18.213538) (end 57.316017 20.925029) (width 0.8) (layer "F.Cu") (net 3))
 (segment (start 57.316017 20.925029) (end 57.316017 23.785057) (width 0.8) (layer "F.Cu") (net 3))
 (segment (start 52.198057 25.817057) (end 50.679057 25.817057) (width 0.8) (layer "F.Cu") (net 3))
 (segment (start 58.315537 21.339043) (end 58.315537 27.827577) (width 0.8) (layer "F.Cu") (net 15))
 (segment (start 52.452057 31.151057) (end 50.679057 31.151057) (width 0.8) (layer "F.Cu") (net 15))
 (segment (start 60.441523 19.213057) (end 58.315537 21.339043) (width 0.8) (layer "F.Cu") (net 15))
 (segment (start 64.881577 29.876057) (end 63.870577 28.865057) (width 0.8) (layer "F.Cu") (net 15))
 (segment (start 58.315537 27.827577) (end 53.722057 32.421057) (width 0.8) (layer "F.Cu") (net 15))
 (segment (start 63.870577 28.865057) (end 63.870576 20.959544) (width 0.8) (layer "F.Cu") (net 15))
 (segment (start 66.935057 29.876057) (end 64.881577 29.876057) (width 0.8) (layer "F.Cu") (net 15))
 (segment (start 53.722057 32.421057) (end 52.452057 31.151057) (width 0.8) (layer "F.Cu") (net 15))
 (segment (start 63.870576 20.959544) (end 62.124089 19.213057) (width 0.8) (layer "F.Cu") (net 15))
 (segment (start 62.124089 19.213057) (end 60.441523 19.213057) (width 0.8) (layer "F.Cu") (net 15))
 (segment (start 66.935057 32.416057) (end 64.136057 32.416057) (width 0.8) (layer "F.Cu") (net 14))
 (segment (start 55.251057 37.755057) (end 53.722057 37.755057) (width 0.8) (layer "F.Cu") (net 14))
 (segment (start 62.871057 31.151057) (end 62.871057 21.373559) (width 0.8) (layer "F.Cu") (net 14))
 (segment (start 59.315057 21.753057) (end 59.315057 33.691057) (width 0.8) (layer "F.Cu") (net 14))
 (segment (start 61.726555 20.229057) (end 60.839057 20.229057) (width 0.8) (layer "F.Cu") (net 14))
 (segment (start 62.871057 21.373559) (end 61.726555 20.229057) (width 0.8) (layer "F.Cu") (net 14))
 (segment (start 53.722057 37.755057) (end 52.452057 36.485057) (width 0.8) (layer "F.Cu") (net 14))
 (segment (start 52.452057 36.485057) (end 50.679057 36.485057) (width 0.8) (layer "F.Cu") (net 14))
 (segment (start 59.315057 33.691057) (end 55.251057 37.755057) (width 0.8) (layer "F.Cu") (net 14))
 (segment (start 60.839057 20.229057) (end 59.315057 21.753057) (width 0.8) (layer "F.Cu") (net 14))
 (segment (start 64.136057 32.416057) (end 62.871057 31.151057) (width 0.8) (layer "F.Cu") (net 14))
 (segment (start 20.662171 26.280171) (end 19.691057 25.309057) (width 0.8) (layer "F.Cu") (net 9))
 (segment (start 22.614213 28.311256) (end 22.5 28.197043) (width 0.8) (layer "F.Cu") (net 9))
 (segment (start 22.485057 26.280171) (end 20.707057 26.280171) (width 0.8) (layer "F.Cu") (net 9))
 (segment (start 25.279057 35.723057) (end 24.737271 35.723057) (width 0.8) (layer "F.Cu") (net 9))
 (segment (start 22.485057 28.197043) (end 22.5 28.197043) (width 0.8) (layer "F.Cu") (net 9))
 (segment (start 25.279057 35.723057) (end 27.321057 37.765057) (width 0.8) (layer "F.Cu") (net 9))
 (segment (start 20.707057 26.280171) (end 19.691057 27.296171) (width 0.8) (layer "F.Cu") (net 9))
 (segment (start 19.691057 25.309057) (end 19.691057 23.755171) (width 0.8) (layer "F.Cu") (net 9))
 (segment (start 22.614213 33.599999) (end 22.614213 28.311256) (width 0.8) (layer "F.Cu") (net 9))
 (segment (start 20.707057 26.280171) (end 20.662171 26.280171) (width 0.8) (layer "F.Cu") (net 9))
 (segment (start 22.5 28.197043) (end 22.579043 28.197043) (width 0.8) (layer "F.Cu") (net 9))
 (segment (start 22.485057 26.280171) (end 22.485057 28.197043) (width 0.8) (layer "F.Cu") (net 9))
 (segment (start 24.737271 35.723057) (end 22.614213 33.599999) (width 0.8) (layer "F.Cu") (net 9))
 (segment (start 24.5 32.7) (end 27.306114 32.7) (width 0.8) (layer "F.Cu") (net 16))
 (segment (start 27.306114 32.7) (end 27.321057 32.685057) (width 0.8) (layer "F.Cu") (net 16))
 (segment (start 23.884568 25.408682) (end 19.691057 21.215171) (width 0.8) (layer "F.Cu") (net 12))
 (segment (start 27.565057 28.611057) (end 25.533057 28.611057) (width 0.8) (layer "F.Cu") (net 12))
 (segment (start 30.283537 21.320577) (end 30.283537 25.892577) (width 0.8) (layer "F.Cu") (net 12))
 (segment (start 31.883057 19.721057) (end 30.283537 21.320577) (width 0.8) (layer "F.Cu") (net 12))
 (segment (start 30.283537 25.892577) (end 27.565057 28.611057) (width 0.8) (layer "F.Cu") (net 12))
 (segment (start 23.884568 26.962568) (end 23.884568 25.408682) (width 0.8) (layer "F.Cu") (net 12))
 (segment (start 25.533057 28.611057) (end 23.884568 26.962568) (width 0.8) (layer "F.Cu") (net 12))
 (segment (start 46.975057 21.605057) (end 46.869057 21.499057) (width 0.8) (layer "F.Cu") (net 13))
 (segment (start 50.679057 21.605057) (end 46.975057 21.605057) (width 0.8) (layer "F.Cu") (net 13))
 (segment (start 50.679057 27.087057) (end 46.869057 27.087057) (width 0.8) (layer "F.Cu") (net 2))
 (segment (start 30.088577 38.39028) (end 28.314769 40.164088) (width 0.8) (layer "F.Cu") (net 10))
 (segment (start 39.249057 25.055057) (end 39.249057 21.499057) (width 0.8) (layer "F.Cu") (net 10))
 (segment (start 30.088577 37.537537) (end 30.088577 38.39028) (width 0.8) (layer "F.Cu") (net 10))
 (segment (start 21.079428 34.916171) (end 19.691057 34.916171) (width 0.8) (layer "F.Cu") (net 10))
 (segment (start 36.455057 27.849057) (end 39.249057 25.055057) (width 0.8) (layer "F.Cu") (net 10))
 (segment (start 34.941057 32.685057) (end 36.455057 31.171057) (width 0.8) (layer "F.Cu") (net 10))
 (segment (start 34.941057 32.685057) (end 30.088577 37.537537) (width 0.8) (layer "F.Cu") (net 10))
 (segment (start 28.314769 40.164088) (end 26.327345 40.164088) (width 0.8) (layer "F.Cu") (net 10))
 (segment (start 26.327345 40.164088) (end 21.079428 34.916171) (width 0.8) (layer "F.Cu") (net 10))
 (segment (start 36.455057 31.171057) (end 36.455057 27.849057) (width 0.8) (layer "F.Cu") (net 10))
 (segment (start 39.249057 27.087057) (end 37.454577 28.881537) (width 0.8) (layer "F.Cu") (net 11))
 (segment (start 29.002506 41.163608) (end 23.398494 41.163608) (width 0.8) (layer "F.Cu") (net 11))
 (segment (start 37.454576 31.585072) (end 36.536824 32.502824) (width 0.8) (layer "F.Cu") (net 11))
 (segment (start 36.536824 32.502824) (end 36.536824 33.62929) (width 0.8) (layer "F.Cu") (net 11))
 (segment (start 37.454577 28.881537) (end 37.454576 31.585072) (width 0.8) (layer "F.Cu") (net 11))
 (segment (start 34.941057 35.225057) (end 29.002506 41.163608) (width 0.8) (layer "F.Cu") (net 11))
 (segment (start 36.536824 33.62929) (end 34.941057 35.225057) (width 0.8) (layer "F.Cu") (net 11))
 (segment (start 23.398494 41.163608) (end 19.691057 37.456171) (width 0.8) (layer "F.Cu") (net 11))
 (segment (start 37.725057 33.945057) (end 39.249057 32.421057) (width 0.8) (layer "F.Cu") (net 7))
 (segment (start 34.941057 37.765057) (end 34.941057 37.237057) (width 0.8) (layer "F.Cu") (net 7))
 (segment (start 34.941057 37.237057) (end 37.725057 34.453057) (width 0.8) (layer "F.Cu") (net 7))
 (segment (start 37.725057 34.453057) (end 37.725057 33.945057) (width 0.8) (layer "F.Cu") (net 7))
 (segment (start 32.542027 27.444087) (end 35.850506 24.135608) (width 0.8) (layer "F.Cu") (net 4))
 (segment (start 35.850508 20.091329) (end 37.96582 17.976017) (width 0.8) (layer "F.Cu") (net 4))
 (segment (start 40.532294 17.976017) (end 43.468948 20.912671) (width 0.8) (layer "F.Cu") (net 4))
 (segment (start 43.468948 33.535166) (end 39.249057 37.755057) (width 0.8) (layer "F.Cu") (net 4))
 (segment (start 32.542026 31.508088) (end 32.542027 27.444087) (width 0.8) (layer "F.Cu") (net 4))
 (segment (start 28.825057 35.225057) (end 32.542026 31.508088) (width 0.8) (layer "F.Cu") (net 4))
 (segment (start 35.850506 24.135608) (end 35.850508 20.091329) (width 0.8) (layer "F.Cu") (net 4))
 (segment (start 43.468948 20.912671) (end 43.468948 33.535166) (width 0.8) (layer "F.Cu") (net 4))
 (segment (start 27.321057 35.225057) (end 28.825057 35.225057) (width 0.8) (layer "F.Cu") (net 4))
 (segment (start 37.96582 17.976017) (end 40.532294 17.976017) (width 0.8) (layer "F.Cu") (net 4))
 (segment (start 50.679057 32.421057) (end 46.869057 32.421057) (width 0.8) (layer "F.Cu") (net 8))
 (segment (start 50.679057 37.755057) (end 46.869057 37.755057) (width 0.8) (layer "F.Cu") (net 5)))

